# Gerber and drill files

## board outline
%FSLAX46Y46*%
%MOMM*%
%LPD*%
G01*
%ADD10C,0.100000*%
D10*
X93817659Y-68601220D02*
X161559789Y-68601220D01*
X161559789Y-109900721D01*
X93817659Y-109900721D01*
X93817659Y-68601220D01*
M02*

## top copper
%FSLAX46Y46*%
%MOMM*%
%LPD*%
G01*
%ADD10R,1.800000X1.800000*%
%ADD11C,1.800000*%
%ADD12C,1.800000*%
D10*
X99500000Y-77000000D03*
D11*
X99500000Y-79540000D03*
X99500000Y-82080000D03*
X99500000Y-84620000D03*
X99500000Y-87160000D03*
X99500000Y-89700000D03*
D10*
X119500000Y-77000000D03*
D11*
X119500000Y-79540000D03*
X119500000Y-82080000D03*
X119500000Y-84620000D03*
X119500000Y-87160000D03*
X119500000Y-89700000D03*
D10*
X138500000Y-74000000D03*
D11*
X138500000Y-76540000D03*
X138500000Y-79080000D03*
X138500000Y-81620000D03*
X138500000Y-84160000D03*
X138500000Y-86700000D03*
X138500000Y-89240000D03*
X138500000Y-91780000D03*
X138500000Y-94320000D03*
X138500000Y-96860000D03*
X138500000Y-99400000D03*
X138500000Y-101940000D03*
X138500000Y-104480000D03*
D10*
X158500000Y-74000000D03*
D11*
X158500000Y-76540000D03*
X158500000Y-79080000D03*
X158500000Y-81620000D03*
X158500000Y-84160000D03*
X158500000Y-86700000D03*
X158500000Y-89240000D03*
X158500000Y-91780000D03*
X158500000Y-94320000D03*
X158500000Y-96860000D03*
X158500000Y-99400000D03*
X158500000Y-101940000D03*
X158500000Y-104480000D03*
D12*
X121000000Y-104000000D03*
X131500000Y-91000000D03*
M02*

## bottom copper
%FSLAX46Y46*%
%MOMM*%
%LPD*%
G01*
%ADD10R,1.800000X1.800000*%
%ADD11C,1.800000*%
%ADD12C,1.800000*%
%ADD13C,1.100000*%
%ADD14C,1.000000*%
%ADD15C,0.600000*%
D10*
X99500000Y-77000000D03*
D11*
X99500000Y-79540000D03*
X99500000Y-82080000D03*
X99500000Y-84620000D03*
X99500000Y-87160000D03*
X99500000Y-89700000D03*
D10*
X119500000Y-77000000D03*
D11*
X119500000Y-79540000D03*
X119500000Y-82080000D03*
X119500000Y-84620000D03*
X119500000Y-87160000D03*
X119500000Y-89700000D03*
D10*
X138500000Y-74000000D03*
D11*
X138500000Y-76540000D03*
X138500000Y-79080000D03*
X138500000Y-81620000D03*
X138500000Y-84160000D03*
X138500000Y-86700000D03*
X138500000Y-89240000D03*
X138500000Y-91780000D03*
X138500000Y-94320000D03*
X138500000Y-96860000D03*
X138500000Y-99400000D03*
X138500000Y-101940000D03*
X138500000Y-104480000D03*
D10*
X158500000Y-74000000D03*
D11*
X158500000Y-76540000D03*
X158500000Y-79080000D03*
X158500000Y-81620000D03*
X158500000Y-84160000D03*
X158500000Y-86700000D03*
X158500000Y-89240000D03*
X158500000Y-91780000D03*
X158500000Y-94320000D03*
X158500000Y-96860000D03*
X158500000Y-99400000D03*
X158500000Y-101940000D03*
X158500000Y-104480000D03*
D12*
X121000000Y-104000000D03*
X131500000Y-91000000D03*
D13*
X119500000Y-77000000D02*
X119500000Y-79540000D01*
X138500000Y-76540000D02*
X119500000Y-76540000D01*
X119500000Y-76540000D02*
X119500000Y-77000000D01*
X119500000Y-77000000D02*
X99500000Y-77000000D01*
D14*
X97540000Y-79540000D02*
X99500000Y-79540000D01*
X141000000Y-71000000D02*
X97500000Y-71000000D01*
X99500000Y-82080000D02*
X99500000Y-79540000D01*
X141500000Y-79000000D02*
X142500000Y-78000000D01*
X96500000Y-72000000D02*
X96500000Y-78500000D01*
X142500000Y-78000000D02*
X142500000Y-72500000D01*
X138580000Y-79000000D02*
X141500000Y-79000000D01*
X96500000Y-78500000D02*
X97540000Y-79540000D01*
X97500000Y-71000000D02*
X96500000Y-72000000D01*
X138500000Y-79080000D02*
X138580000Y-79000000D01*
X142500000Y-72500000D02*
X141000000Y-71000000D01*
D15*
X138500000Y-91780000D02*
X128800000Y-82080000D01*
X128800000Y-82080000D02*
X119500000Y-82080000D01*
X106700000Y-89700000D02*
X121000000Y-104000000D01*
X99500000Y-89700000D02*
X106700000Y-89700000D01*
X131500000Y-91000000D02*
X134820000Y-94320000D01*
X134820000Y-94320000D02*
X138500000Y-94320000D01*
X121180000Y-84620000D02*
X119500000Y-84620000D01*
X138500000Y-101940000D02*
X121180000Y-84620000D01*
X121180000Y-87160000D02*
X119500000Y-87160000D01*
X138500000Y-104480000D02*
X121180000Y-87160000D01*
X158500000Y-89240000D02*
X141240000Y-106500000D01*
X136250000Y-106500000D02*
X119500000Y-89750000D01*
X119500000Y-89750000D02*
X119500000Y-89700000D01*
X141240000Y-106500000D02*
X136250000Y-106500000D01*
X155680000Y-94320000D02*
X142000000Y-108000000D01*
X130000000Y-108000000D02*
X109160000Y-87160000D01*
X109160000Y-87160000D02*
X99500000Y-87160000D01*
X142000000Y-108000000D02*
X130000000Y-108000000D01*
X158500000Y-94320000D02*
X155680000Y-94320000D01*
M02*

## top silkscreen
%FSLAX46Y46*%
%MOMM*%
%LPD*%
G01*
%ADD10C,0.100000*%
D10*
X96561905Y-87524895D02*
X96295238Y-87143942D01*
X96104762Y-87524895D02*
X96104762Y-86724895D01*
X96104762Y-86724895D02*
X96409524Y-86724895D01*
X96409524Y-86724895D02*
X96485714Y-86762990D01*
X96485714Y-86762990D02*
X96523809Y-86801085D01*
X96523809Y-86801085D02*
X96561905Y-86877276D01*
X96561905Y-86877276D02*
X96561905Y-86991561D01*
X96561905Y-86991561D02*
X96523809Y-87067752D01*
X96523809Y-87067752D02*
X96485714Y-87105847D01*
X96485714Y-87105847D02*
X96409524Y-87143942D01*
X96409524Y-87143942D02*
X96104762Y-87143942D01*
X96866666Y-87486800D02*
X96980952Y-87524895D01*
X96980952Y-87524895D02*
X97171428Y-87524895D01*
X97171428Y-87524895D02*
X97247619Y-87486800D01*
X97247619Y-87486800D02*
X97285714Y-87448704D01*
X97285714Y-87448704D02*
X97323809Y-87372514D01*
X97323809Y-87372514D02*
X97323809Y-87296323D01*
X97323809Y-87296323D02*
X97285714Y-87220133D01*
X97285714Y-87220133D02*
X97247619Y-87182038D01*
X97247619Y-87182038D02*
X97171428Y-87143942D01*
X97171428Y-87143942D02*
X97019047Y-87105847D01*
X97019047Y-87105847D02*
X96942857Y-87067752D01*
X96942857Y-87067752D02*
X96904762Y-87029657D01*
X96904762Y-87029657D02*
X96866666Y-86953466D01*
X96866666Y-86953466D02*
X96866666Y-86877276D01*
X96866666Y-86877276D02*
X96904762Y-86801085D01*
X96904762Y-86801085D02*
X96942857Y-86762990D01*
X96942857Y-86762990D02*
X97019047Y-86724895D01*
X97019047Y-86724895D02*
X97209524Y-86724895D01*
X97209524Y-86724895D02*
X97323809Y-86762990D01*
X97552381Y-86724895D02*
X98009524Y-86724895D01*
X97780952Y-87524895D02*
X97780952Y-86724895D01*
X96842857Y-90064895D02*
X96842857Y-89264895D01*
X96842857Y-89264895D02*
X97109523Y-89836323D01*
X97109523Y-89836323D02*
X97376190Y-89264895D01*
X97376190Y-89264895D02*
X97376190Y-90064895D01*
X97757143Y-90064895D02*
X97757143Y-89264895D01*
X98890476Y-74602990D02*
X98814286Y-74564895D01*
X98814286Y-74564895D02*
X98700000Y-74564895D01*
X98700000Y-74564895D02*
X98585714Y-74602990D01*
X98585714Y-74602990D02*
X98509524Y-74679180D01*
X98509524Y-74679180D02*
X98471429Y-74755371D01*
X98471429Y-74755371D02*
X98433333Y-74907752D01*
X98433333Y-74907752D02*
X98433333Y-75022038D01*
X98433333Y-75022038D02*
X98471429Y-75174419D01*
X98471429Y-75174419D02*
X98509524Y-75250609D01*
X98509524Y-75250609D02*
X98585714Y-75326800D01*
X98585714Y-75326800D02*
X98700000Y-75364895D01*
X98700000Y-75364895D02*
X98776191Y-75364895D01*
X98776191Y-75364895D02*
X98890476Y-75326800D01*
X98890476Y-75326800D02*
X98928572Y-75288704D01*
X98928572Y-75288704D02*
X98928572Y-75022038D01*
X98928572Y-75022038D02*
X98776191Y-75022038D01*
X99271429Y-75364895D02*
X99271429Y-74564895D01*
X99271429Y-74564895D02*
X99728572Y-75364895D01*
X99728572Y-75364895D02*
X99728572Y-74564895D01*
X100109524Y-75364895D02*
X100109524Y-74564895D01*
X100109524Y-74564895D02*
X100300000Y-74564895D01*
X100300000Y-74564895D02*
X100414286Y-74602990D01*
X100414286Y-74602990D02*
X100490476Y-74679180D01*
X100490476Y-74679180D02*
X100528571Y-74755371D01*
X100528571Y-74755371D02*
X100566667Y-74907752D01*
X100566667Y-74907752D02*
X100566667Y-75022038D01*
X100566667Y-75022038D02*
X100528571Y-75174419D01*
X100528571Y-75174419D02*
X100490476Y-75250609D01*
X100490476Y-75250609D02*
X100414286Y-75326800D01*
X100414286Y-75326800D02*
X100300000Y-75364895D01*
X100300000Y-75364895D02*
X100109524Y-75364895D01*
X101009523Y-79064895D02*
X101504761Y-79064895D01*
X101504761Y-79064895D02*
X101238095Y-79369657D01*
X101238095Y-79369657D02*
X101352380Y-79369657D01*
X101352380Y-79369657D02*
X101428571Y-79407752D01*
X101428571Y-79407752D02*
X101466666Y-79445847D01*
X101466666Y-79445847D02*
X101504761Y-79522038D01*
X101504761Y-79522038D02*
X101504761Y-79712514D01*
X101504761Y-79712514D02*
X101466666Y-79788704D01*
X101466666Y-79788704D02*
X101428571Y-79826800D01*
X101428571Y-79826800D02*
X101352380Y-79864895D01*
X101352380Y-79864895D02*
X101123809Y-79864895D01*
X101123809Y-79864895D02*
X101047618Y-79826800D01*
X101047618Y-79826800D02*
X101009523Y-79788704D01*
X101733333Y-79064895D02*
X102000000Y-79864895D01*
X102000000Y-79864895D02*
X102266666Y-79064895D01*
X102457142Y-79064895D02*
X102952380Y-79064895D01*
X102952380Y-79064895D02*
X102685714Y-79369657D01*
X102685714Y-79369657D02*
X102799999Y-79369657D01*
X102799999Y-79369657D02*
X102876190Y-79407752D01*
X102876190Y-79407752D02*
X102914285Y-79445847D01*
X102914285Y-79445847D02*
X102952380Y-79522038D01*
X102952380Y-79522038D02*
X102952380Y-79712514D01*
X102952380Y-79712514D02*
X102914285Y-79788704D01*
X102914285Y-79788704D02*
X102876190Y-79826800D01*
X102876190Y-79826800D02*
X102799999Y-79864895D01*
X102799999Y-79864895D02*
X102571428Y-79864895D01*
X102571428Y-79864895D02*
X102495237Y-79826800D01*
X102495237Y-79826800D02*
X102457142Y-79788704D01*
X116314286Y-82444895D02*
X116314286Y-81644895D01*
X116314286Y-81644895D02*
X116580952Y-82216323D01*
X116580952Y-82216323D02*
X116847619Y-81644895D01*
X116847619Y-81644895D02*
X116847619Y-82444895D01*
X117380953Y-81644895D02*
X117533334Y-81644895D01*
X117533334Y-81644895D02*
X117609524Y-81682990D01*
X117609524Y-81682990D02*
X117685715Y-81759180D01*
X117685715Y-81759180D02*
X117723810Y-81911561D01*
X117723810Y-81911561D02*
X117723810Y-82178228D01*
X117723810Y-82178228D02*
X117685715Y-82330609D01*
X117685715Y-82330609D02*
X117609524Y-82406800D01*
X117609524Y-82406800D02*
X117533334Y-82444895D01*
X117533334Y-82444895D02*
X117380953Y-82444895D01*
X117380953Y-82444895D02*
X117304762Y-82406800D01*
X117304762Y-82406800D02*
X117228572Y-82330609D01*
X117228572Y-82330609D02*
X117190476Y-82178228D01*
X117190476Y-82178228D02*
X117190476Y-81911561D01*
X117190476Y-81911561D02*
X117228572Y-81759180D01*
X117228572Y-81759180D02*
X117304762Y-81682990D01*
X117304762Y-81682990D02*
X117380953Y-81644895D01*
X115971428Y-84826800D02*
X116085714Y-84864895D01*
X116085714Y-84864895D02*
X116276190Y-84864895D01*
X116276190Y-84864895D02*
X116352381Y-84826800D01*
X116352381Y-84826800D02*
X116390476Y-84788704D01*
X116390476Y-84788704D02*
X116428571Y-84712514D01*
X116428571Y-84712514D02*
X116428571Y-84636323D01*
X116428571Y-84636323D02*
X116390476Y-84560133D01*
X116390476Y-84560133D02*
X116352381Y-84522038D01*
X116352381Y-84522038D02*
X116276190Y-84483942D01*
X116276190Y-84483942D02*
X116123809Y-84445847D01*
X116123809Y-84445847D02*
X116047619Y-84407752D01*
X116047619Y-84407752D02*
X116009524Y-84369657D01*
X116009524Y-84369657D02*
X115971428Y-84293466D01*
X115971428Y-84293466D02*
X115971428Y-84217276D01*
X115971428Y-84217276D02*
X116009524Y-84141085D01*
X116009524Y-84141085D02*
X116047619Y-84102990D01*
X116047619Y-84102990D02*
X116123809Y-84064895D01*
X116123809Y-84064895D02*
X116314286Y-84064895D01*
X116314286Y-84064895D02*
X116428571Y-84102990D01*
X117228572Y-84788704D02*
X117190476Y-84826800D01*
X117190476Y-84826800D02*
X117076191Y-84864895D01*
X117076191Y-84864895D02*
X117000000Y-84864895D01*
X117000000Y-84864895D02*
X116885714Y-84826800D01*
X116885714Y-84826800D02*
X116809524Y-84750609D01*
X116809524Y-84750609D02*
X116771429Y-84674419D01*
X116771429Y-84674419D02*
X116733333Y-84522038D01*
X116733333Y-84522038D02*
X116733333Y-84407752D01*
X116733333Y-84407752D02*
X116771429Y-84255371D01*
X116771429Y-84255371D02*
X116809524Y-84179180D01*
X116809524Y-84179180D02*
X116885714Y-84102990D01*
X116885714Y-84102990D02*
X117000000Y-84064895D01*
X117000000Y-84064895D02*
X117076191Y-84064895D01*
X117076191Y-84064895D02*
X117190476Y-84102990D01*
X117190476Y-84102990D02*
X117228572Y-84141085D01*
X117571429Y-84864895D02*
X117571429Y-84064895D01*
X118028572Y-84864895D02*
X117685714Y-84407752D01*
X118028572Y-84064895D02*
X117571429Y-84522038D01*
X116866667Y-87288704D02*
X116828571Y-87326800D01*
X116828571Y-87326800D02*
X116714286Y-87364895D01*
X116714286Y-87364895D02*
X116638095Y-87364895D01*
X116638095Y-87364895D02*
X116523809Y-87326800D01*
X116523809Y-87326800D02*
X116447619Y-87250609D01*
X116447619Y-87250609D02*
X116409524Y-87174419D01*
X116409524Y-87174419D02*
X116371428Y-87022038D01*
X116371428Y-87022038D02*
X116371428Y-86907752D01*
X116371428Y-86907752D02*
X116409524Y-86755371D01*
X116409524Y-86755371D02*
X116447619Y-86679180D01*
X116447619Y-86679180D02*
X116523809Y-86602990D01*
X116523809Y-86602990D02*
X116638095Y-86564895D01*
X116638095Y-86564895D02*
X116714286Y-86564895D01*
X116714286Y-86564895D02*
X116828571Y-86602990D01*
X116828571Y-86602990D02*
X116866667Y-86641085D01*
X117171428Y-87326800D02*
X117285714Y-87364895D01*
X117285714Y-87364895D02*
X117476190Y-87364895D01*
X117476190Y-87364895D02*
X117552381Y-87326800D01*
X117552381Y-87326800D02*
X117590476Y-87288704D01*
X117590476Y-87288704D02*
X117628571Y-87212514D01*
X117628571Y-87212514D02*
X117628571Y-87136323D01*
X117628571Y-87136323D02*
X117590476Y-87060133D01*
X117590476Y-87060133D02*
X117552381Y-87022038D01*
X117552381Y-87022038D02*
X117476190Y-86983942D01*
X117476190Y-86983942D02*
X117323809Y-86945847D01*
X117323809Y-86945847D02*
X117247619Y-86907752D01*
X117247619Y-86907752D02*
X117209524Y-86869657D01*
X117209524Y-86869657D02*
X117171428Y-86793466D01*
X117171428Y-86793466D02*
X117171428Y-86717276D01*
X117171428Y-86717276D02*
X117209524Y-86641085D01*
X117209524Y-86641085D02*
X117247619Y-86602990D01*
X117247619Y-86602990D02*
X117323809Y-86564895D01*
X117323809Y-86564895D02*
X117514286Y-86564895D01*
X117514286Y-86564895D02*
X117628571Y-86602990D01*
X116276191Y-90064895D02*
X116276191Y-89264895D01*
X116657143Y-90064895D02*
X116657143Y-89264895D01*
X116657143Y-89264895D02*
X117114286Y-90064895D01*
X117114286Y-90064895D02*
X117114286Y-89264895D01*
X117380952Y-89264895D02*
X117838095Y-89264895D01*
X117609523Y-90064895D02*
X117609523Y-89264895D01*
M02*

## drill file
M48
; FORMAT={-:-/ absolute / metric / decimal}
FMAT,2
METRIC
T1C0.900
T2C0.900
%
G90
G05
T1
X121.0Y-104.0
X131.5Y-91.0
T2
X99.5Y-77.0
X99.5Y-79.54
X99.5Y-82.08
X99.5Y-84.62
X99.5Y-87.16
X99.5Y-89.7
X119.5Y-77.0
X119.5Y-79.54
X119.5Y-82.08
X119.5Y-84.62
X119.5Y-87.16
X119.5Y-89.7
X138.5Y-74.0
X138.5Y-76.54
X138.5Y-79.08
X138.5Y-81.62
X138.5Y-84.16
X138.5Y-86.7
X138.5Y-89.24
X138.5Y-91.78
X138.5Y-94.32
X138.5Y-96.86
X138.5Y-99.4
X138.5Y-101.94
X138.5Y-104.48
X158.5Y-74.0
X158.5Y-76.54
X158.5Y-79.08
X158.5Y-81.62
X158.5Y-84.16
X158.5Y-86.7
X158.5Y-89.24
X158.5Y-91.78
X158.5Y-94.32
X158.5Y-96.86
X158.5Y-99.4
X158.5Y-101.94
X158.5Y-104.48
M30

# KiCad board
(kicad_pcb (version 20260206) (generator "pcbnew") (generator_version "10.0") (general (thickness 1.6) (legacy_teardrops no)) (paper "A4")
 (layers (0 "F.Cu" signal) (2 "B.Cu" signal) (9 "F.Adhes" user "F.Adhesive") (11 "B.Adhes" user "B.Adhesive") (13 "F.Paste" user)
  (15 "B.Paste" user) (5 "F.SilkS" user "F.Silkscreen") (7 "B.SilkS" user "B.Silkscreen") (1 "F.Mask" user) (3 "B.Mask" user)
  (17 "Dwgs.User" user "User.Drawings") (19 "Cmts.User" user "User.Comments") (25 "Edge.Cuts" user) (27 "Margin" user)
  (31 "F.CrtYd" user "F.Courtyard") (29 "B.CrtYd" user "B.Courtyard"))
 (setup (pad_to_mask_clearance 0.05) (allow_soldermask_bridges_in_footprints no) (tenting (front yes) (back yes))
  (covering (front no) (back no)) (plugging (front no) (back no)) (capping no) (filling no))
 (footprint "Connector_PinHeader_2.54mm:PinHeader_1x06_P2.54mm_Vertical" (layer "F.Cu") (at 99.5 77)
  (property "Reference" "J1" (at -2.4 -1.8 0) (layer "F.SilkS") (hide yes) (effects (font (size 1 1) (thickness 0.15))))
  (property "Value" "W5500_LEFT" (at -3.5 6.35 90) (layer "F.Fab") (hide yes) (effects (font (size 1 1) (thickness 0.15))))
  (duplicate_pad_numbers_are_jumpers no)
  (pad "1" thru_hole rect (at 0 0) (size 1.8 1.8) (drill 0.9) (layers "*.Cu" "*.Mask") (remove_unused_layers no) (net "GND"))
  (pad "2" thru_hole circle (at 0 2.54) (size 1.8 1.8) (drill 0.9) (layers "*.Cu" "*.Mask") (remove_unused_layers no) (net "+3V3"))
  (pad "3" thru_hole circle (at 0 5.08) (size 1.8 1.8) (drill 0.9) (layers "*.Cu" "*.Mask") (remove_unused_layers no) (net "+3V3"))
  (pad "4" thru_hole circle (at 0 7.62) (size 1.8 1.8) (drill 0.9) (layers "*.Cu" "*.Mask") (remove_unused_layers no))
  (pad "5" thru_hole circle (at 0 10.16) (size 1.8 1.8) (drill 0.9) (layers "*.Cu" "*.Mask") (remove_unused_layers no) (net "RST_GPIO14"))
  (pad "6" thru_hole circle (at 0 12.7) (size 1.8 1.8) (drill 0.9) (layers "*.Cu" "*.Mask") (remove_unused_layers no) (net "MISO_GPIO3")))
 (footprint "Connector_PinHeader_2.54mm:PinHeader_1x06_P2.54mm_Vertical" (layer "F.Cu") (at 119.5 77)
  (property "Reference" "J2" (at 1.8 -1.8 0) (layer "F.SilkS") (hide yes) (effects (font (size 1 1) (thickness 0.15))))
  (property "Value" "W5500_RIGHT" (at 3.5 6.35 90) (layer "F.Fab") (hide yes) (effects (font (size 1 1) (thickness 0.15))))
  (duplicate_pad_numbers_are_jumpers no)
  (pad "1" thru_hole rect (at 0 0) (size 1.8 1.8) (drill 0.9) (layers "*.Cu" "*.Mask") (remove_unused_layers no) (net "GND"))
  (pad "2" thru_hole circle (at 0 2.54) (size 1.8 1.8) (drill 0.9) (layers "*.Cu" "*.Mask") (remove_unused_layers no) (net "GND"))
  (pad "3" thru_hole circle (at 0 5.08) (size 1.8 1.8) (drill 0.9) (layers "*.Cu" "*.Mask") (remove_unused_layers no) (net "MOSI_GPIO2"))
  (pad "4" thru_hole circle (at 0 7.62) (size 1.8 1.8) (drill 0.9) (layers "*.Cu" "*.Mask") (remove_unused_layers no) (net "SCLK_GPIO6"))
  (pad "5" thru_hole circle (at 0 10.16) (size 1.8 1.8) (drill 0.9) (layers "*.Cu" "*.Mask") (remove_unused_layers no) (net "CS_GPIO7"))
  (pad "6" thru_hole circle (at 0 12.7) (size 1.8 1.8) (drill 0.9) (layers "*.Cu" "*.Mask") (remove_unused_layers no) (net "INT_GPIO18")))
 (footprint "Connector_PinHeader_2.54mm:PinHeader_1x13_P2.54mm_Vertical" (layer "F.Cu") (at 138.5 74)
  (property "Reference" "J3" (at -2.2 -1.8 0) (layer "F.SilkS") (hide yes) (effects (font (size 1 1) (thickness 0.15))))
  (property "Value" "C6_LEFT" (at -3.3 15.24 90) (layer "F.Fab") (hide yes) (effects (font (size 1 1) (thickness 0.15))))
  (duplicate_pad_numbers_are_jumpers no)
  (pad "1" thru_hole rect (at 0 0) (size 1.8 1.8) (drill 0.9) (layers "*.Cu" "*.Mask") (remove_unused_layers no) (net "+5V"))
  (pad "2" thru_hole circle (at 0 2.54) (size 1.8 1.8) (drill 0.9) (layers "*.Cu" "*.Mask") (remove_unused_layers no) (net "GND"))
  (pad "3" thru_hole circle (at 0 5.08) (size 1.8 1.8) (drill 0.9) (layers "*.Cu" "*.Mask") (remove_unused_layers no) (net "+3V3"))
  (pad "4" thru_hole circle (at 0 7.62) (size 1.8 1.8) (drill 0.9) (layers "*.Cu" "*.Mask") (remove_unused_layers no))
  (pad "5" thru_hole circle (at 0 10.16) (size 1.8 1.8) (drill 0.9) (layers "*.Cu" "*.Mask") (remove_unused_layers no))
  (pad "6" thru_hole circle (at 0 12.7) (size 1.8 1.8) (drill 0.9) (layers "*.Cu" "*.Mask") (remove_unused_layers no))
  (pad "7" thru_hole circle (at 0 15.24) (size 1.8 1.8) (drill 0.9) (layers "*.Cu" "*.Mask") (remove_unused_layers no))
  (pad "8" thru_hole circle (at 0 17.78) (size 1.8 1.8) (drill 0.9) (layers "*.Cu" "*.Mask") (remove_unused_layers no) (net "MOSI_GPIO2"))
  (pad "9" thru_hole circle (at 0 20.32) (size 1.8 1.8) (drill 0.9) (layers "*.Cu" "*.Mask") (remove_unused_layers no) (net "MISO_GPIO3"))
  (pad "10" thru_hole circle (at 0 22.86) (size 1.8 1.8) (drill 0.9) (layers "*.Cu" "*.Mask") (remove_unused_layers no))
  (pad "11" thru_hole circle (at 0 25.4) (size 1.8 1.8) (drill 0.9) (layers "*.Cu" "*.Mask") (remove_unused_layers no))
  (pad "12" thru_hole circle (at 0 27.94) (size 1.8 1.8) (drill 0.9) (layers "*.Cu" "*.Mask") (remove_unused_layers no) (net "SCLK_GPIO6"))
  (pad "13" thru_hole circle (at 0 30.48) (size 1.8 1.8) (drill 0.9) (layers "*.Cu" "*.Mask") (remove_unused_layers no) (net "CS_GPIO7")))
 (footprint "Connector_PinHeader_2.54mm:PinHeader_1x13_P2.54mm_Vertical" (layer "F.Cu") (at 158.5 74)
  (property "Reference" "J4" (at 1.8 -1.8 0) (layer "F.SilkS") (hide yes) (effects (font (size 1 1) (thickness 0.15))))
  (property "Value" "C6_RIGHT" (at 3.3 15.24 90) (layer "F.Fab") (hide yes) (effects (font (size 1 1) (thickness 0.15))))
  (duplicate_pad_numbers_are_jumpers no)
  (pad "1" thru_hole rect (at 0 0) (size 1.8 1.8) (drill 0.9) (layers "*.Cu" "*.Mask") (remove_unused_layers no))
  (pad "2" thru_hole circle (at 0 2.54) (size 1.8 1.8) (drill 0.9) (layers "*.Cu" "*.Mask") (remove_unused_layers no))
  (pad "3" thru_hole circle (at 0 5.08) (size 1.8 1.8) (drill 0.9) (layers "*.Cu" "*.Mask") (remove_unused_layers no))
  (pad "4" thru_hole circle (at 0 7.62) (size 1.8 1.8) (drill 0.9) (layers "*.Cu" "*.Mask") (remove_unused_layers no))
  (pad "5" thru_hole circle (at 0 10.16) (size 1.8 1.8) (drill 0.9) (layers "*.Cu" "*.Mask") (remove_unused_layers no))
  (pad "6" thru_hole circle (at 0 12.7) (size 1.8 1.8) (drill 0.9) (layers "*.Cu" "*.Mask") (remove_unused_layers no))
  (pad "7" thru_hole circle (at 0 15.24) (size 1.8 1.8) (drill 0.9) (layers "*.Cu" "*.Mask") (remove_unused_layers no) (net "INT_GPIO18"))
  (pad "8" thru_hole circle (at 0 17.78) (size 1.8 1.8) (drill 0.9) (layers "*.Cu" "*.Mask") (remove_unused_layers no))
  (pad "9" thru_hole circle (at 0 20.32) (size 1.8 1.8) (drill 0.9) (layers "*.Cu" "*.Mask") (remove_unused_layers no) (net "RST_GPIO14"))
  (pad "10" thru_hole circle (at 0 22.86) (size 1.8 1.8) (drill 0.9) (layers "*.Cu" "*.Mask") (remove_unused_layers no))
  (pad "11" thru_hole circle (at 0 25.4) (size 1.8 1.8) (drill 0.9) (layers "*.Cu" "*.Mask") (remove_unused_layers no))
  (pad "12" thru_hole circle (at 0 27.94) (size 1.8 1.8) (drill 0.9) (layers "*.Cu" "*.Mask") (remove_unused_layers no))
  (pad "13" thru_hole circle (at 0 30.48) (size 1.8 1.8) (drill 0.9) (layers "*.Cu" "*.Mask") (remove_unused_layers no)))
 (gr_rect (start 93.817659 68.60122) (end 161.559789 109.900721) (stroke (width 0.1) (type solid)) (fill no) (layer "Edge.Cuts"))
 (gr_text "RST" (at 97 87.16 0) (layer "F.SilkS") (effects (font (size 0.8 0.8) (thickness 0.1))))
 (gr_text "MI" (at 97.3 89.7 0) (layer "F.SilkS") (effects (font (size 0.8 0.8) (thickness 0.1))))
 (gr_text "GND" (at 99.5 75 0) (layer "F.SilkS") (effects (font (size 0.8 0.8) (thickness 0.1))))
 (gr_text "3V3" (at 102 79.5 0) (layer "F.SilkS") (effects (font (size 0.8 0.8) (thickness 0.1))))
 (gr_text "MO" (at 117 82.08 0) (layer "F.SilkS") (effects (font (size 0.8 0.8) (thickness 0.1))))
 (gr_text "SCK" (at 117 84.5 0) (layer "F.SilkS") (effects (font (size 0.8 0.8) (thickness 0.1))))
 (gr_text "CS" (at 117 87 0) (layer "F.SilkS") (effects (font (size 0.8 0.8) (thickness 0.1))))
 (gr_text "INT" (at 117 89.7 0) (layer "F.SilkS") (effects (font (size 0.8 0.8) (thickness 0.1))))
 (segment (start 119.5 77) (end 119.5 79.54) (width 1.1) (layer "B.Cu") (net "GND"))
 (segment (start 138.5 76.54) (end 119.5 76.54) (width 1.1) (layer "B.Cu") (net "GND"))
 (segment (start 119.5 76.54) (end 119.5 77) (width 1.1) (layer "B.Cu") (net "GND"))
 (segment (start 119.5 77) (end 99.5 77) (width 1.1) (layer "B.Cu") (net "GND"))
 (segment (start 97.54 79.54) (end 99.5 79.54) (width 1) (layer "B.Cu") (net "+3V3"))
 (segment (start 141 71) (end 97.5 71) (width 1) (layer "B.Cu") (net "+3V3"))
 (segment (start 99.5 82.08) (end 99.5 79.54) (width 1) (layer "B.Cu") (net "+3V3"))
 (segment (start 141.5 79) (end 142.5 78) (width 1) (layer "B.Cu") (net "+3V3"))
 (segment (start 96.5 72) (end 96.5 78.5) (width 1) (layer "B.Cu") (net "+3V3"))
 (segment (start 142.5 78) (end 142.5 72.5) (width 1) (layer "B.Cu") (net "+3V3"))
 (segment (start 138.58 79) (end 141.5 79) (width 1) (layer "B.Cu") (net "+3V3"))
 (segment (start 96.5 78.5) (end 97.54 79.54) (width 1) (layer "B.Cu") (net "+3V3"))
 (segment (start 97.5 71) (end 96.5 72) (width 1) (layer "B.Cu") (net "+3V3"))
 (segment (start 138.5 79.08) (end 138.58 79) (width 1) (layer "B.Cu") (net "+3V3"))
 (segment (start 142.5 72.5) (end 141 71) (width 1) (layer "B.Cu") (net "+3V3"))
 (segment (start 138.5 91.78) (end 128.8 82.08) (width 0.6) (layer "B.Cu") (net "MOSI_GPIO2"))
 (segment (start 128.8 82.08) (end 119.5 82.08) (width 0.6) (layer "B.Cu") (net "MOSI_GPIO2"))
 (via (at 121 104) (size 1.8) (drill 0.9) (layers "F.Cu" "B.Cu") (free yes) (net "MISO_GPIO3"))
 (via (at 131.5 91) (size 1.8) (drill 0.9) (layers "F.Cu" "B.Cu") (free yes) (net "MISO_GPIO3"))
 (segment (start 106.7 89.7) (end 121 104) (width 0.6) (layer "B.Cu") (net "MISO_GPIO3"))
 (segment (start 99.5 89.7) (end 106.7 89.7) (width 0.6) (layer "B.Cu") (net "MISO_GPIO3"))
 (segment (start 131.5 91) (end 134.82 94.32) (width 0.6) (layer "B.Cu") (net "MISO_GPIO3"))
 (segment (start 134.82 94.32) (end 138.5 94.32) (width 0.6) (layer "B.Cu") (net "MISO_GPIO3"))
 (segment (start 121.18 84.62) (end 119.5 84.62) (width 0.6) (layer "B.Cu") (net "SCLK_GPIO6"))
 (segment (start 138.5 101.94) (end 121.18 84.62) (width 0.6) (layer "B.Cu") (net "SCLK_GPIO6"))
 (segment (start 121.18 87.16) (end 119.5 87.16) (width 0.6) (layer "B.Cu") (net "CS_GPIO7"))
 (segment (start 138.5 104.48) (end 121.18 87.16) (width 0.6) (layer "B.Cu") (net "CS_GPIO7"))
 (segment (start 158.5 89.24) (end 141.24 106.5) (width 0.6) (layer "B.Cu") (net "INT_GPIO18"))
 (segment (start 136.25 106.5) (end 119.5 89.75) (width 0.6) (layer "B.Cu") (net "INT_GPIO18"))
 (segment (start 119.5 89.75) (end 119.5 89.7) (width 0.6) (layer "B.Cu") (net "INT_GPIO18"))
 (segment (start 141.24 106.5) (end 136.25 106.5) (width 0.6) (layer "B.Cu") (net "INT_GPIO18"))
 (segment (start 155.68 94.32) (end 142 108) (width 0.6) (layer "B.Cu") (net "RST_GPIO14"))
 (segment (start 130 108) (end 109.16 87.16) (width 0.6) (layer "B.Cu") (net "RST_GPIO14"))
 (segment (start 109.16 87.16) (end 99.5 87.16) (width 0.6) (layer "B.Cu") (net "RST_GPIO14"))
 (segment (start 142 108) (end 130 108) (width 0.6) (layer "B.Cu") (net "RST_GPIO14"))
 (segment (start 158.5 94.32) (end 155.68 94.32) (width 0.6) (layer "B.Cu") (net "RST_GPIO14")))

